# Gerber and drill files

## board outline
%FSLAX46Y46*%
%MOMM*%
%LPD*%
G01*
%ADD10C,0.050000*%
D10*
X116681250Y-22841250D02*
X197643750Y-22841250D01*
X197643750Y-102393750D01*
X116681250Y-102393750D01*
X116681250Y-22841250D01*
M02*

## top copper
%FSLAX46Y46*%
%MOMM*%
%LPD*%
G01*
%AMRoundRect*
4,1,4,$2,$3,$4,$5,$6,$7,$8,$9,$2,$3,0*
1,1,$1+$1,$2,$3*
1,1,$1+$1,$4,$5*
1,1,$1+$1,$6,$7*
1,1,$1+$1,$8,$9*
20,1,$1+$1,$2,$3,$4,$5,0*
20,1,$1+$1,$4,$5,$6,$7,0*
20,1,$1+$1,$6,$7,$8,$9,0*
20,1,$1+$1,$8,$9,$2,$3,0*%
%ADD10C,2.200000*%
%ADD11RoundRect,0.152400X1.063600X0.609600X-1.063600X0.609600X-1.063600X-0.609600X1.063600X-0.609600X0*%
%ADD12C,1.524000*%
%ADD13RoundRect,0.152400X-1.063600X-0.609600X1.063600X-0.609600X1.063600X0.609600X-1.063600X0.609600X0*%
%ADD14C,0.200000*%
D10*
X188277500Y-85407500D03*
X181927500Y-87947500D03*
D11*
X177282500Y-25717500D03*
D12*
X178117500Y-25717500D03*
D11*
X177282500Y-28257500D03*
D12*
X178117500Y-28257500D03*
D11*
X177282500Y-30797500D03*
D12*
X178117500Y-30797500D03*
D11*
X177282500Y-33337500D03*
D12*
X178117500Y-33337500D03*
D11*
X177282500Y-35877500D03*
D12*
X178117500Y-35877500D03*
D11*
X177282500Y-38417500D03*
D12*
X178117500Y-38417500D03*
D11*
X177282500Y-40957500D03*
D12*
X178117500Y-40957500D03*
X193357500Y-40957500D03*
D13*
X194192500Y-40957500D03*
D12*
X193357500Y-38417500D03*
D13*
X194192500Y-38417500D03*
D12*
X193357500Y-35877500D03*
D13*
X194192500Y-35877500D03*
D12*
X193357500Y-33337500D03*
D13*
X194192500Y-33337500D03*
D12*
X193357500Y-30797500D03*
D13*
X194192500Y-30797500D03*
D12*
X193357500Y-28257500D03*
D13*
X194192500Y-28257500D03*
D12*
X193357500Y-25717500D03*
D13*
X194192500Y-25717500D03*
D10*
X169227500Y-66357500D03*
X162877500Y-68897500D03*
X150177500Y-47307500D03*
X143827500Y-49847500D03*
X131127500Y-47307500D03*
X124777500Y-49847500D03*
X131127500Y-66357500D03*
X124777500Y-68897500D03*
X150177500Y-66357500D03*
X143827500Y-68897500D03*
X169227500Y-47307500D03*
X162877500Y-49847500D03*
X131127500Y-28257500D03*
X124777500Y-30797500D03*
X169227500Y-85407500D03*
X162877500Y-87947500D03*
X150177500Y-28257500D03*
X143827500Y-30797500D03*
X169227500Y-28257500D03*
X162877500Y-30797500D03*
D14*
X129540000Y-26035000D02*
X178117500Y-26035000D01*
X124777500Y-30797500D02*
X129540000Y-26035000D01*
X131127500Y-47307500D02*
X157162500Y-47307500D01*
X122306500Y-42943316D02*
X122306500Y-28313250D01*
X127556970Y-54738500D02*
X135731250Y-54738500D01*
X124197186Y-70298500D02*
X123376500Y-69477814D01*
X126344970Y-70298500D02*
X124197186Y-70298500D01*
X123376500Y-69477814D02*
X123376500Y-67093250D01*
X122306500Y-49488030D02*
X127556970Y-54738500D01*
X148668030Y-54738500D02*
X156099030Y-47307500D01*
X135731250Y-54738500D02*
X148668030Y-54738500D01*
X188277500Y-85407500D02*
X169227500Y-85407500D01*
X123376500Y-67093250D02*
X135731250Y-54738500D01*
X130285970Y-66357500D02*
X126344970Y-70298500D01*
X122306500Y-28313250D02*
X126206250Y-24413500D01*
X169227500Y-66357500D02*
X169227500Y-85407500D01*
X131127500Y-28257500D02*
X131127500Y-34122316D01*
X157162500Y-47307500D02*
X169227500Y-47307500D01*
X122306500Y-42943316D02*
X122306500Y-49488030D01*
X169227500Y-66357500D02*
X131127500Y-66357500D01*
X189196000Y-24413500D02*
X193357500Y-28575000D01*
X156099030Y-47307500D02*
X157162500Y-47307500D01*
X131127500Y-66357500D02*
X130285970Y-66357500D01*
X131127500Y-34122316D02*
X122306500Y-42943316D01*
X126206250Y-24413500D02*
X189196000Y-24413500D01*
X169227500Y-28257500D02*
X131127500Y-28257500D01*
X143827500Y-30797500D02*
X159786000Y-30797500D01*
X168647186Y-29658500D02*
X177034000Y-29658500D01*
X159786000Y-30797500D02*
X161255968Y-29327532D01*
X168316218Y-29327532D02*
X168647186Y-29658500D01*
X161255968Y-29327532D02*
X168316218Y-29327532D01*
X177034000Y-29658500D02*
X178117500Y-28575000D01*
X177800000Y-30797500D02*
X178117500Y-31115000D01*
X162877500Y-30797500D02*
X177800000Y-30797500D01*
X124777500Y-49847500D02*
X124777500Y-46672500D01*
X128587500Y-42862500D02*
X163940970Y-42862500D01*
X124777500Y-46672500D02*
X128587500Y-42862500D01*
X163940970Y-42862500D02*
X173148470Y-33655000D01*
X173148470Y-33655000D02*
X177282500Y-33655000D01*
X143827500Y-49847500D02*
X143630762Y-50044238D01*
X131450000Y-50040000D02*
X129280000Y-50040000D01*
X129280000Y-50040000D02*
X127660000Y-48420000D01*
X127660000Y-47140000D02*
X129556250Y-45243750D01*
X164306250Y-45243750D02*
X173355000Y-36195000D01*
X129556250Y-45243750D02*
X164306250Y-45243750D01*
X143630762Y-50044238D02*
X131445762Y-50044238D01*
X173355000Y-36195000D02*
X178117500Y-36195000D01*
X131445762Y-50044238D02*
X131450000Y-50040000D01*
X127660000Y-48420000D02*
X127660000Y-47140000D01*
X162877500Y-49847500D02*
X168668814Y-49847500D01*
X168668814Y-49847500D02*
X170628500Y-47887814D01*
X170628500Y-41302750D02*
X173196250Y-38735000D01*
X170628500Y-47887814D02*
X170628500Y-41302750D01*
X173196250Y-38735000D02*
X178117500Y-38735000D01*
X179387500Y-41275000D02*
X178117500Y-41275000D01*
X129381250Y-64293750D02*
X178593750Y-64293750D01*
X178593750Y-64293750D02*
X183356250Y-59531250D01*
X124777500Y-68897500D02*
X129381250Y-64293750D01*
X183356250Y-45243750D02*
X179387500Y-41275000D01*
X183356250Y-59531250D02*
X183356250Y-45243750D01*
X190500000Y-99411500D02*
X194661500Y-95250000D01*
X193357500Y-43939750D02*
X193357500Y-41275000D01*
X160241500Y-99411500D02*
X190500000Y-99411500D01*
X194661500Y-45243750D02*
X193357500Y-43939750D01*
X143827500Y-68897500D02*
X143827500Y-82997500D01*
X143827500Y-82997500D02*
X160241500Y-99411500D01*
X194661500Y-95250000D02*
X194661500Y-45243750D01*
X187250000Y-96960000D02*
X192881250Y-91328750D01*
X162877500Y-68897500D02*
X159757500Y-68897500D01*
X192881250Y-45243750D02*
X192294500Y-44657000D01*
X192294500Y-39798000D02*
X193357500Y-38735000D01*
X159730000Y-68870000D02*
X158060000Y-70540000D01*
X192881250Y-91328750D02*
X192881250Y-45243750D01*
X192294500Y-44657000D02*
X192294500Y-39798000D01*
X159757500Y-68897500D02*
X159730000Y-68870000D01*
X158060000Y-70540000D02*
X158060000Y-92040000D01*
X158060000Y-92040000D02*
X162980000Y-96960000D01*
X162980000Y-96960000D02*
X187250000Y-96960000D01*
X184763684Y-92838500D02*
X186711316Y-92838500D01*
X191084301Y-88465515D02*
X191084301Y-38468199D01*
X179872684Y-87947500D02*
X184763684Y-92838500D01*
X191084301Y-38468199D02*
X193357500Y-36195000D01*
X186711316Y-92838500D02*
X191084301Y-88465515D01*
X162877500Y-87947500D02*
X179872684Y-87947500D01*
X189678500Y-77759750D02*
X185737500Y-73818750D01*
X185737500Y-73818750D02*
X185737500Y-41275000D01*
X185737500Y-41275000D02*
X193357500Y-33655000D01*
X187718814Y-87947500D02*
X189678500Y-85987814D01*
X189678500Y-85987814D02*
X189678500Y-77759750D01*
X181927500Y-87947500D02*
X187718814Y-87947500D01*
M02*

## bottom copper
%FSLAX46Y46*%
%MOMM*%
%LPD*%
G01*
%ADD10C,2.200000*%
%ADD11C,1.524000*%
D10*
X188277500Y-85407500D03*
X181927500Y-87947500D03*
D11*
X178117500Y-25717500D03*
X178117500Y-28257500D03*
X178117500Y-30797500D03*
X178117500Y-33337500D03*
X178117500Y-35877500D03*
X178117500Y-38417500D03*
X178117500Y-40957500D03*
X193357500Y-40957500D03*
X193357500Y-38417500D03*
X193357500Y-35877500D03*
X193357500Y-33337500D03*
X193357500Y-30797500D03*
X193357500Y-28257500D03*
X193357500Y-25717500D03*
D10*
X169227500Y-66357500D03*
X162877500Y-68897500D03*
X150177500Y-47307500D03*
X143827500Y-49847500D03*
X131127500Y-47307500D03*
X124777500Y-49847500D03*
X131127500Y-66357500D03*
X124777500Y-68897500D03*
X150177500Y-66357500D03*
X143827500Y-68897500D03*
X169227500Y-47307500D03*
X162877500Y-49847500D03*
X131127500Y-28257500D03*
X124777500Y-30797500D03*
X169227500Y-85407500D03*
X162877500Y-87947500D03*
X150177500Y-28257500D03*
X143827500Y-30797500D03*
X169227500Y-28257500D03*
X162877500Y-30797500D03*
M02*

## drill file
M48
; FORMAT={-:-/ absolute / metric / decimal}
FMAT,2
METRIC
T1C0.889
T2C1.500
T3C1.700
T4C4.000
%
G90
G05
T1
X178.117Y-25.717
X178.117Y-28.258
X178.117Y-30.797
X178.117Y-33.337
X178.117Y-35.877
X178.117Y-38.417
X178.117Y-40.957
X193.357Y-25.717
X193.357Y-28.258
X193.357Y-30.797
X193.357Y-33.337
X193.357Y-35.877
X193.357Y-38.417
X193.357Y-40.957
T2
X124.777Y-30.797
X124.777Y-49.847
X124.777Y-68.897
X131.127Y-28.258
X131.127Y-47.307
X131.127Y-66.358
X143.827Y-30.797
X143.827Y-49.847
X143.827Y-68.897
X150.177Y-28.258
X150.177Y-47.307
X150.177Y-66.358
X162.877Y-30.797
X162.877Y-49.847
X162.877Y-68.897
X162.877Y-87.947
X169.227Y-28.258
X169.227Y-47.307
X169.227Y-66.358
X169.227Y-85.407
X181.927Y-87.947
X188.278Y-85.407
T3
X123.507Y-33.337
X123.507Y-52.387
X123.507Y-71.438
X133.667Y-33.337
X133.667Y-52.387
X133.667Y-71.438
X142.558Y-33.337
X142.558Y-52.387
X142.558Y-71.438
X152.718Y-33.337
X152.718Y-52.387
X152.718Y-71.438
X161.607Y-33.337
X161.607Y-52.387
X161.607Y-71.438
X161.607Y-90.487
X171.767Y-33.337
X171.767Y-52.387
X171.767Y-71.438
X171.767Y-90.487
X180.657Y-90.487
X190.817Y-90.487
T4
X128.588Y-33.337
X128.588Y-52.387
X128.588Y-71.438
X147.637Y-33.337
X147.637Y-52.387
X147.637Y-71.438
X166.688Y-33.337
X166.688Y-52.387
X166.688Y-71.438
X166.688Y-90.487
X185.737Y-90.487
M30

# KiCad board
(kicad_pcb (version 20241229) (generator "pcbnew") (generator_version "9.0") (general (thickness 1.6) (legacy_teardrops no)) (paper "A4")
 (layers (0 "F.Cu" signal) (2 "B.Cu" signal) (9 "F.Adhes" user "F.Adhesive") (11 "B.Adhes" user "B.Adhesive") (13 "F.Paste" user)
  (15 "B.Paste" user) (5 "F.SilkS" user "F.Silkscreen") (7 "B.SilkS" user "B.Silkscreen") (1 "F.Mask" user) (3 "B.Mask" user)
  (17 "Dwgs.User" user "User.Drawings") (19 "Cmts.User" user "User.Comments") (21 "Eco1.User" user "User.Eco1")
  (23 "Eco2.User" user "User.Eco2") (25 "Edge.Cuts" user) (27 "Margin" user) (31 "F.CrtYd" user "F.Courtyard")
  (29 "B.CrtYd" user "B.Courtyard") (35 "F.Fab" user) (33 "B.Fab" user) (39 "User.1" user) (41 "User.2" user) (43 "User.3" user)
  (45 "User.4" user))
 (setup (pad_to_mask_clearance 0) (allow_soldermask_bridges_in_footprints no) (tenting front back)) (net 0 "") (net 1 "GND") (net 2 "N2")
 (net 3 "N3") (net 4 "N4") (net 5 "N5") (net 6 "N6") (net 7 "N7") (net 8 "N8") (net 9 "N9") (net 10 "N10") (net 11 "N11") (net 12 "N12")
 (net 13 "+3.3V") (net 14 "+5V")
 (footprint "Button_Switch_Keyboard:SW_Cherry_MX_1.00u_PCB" (layer "F.Cu") (at 188.2775 85.4075)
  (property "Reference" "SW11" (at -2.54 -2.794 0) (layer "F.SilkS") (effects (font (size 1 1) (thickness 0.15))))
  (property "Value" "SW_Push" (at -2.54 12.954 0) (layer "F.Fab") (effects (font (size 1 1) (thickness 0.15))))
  (pad "" np_thru_hole circle (at -7.62 5.08) (size 1.7 1.7) (drill 1.7) (layers "*.Cu" "*.Mask"))
  (pad "" np_thru_hole circle (at -2.54 5.08) (size 4 4) (drill 4) (layers "*.Cu" "*.Mask"))
  (pad "" np_thru_hole circle (at 2.54 5.08) (size 1.7 1.7) (drill 1.7) (layers "*.Cu" "*.Mask"))
  (pad "1" thru_hole circle (at 0 0) (size 2.2 2.2) (drill 1.5) (layers "*.Cu" "*.Mask") (remove_unused_layers no) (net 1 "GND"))
  (pad "2" thru_hole circle (at -6.35 2.54) (size 2.2 2.2) (drill 1.5) (layers "*.Cu" "*.Mask") (remove_unused_layers no) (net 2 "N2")))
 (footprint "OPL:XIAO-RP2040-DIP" (layer "F.Cu") (at 185.7375 33.3375)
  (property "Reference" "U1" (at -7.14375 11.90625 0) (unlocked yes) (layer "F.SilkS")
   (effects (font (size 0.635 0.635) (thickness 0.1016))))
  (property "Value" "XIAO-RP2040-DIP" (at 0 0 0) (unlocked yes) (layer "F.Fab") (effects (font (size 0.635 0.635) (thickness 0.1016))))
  (pad "1" smd roundrect (at -8.455 -7.62 180) (size 2.432 1.524) (layers "F.Cu" "F.Mask") (roundrect_rratio 0.1) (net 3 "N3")
   (thermal_bridge_angle 45))
  (pad "1" thru_hole circle (at -7.62 -7.62 180) (size 1.524 1.524) (drill 0.889) (layers "*.Cu" "*.Mask") (remove_unused_layers no)
   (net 3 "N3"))
  (pad "2" smd roundrect (at -8.455 -5.08 180) (size 2.432 1.524) (layers "F.Cu" "F.Mask") (roundrect_rratio 0.1) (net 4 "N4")
   (thermal_bridge_angle 45))
  (pad "2" thru_hole circle (at -7.62 -5.08 180) (size 1.524 1.524) (drill 0.889) (layers "*.Cu" "*.Mask") (remove_unused_layers no)
   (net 4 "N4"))
  (pad "3" smd roundrect (at -8.455 -2.54 180) (size 2.432 1.524) (layers "F.Cu" "F.Mask") (roundrect_rratio 0.1) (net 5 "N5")
   (thermal_bridge_angle 45))
  (pad "3" thru_hole circle (at -7.62 -2.54 180) (size 1.524 1.524) (drill 0.889) (layers "*.Cu" "*.Mask") (remove_unused_layers no)
   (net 5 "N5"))
  (pad "4" smd roundrect (at -8.455 0 180) (size 2.432 1.524) (layers "F.Cu" "F.Mask") (roundrect_rratio 0.1) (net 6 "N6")
   (thermal_bridge_angle 45))
  (pad "4" thru_hole circle (at -7.62 0 180) (size 1.524 1.524) (drill 0.889) (layers "*.Cu" "*.Mask") (remove_unused_layers no)
   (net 6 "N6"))
  (pad "5" smd roundrect (at -8.455 2.54 180) (size 2.432 1.524) (layers "F.Cu" "F.Mask") (roundrect_rratio 0.1) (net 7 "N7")
   (thermal_bridge_angle 45))
  (pad "5" thru_hole circle (at -7.62 2.54 180) (size 1.524 1.524) (drill 0.889) (layers "*.Cu" "*.Mask") (remove_unused_layers no)
   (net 7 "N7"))
  (pad "6" smd roundrect (at -8.455 5.08 180) (size 2.432 1.524) (layers "F.Cu" "F.Mask") (roundrect_rratio 0.1) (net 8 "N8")
   (thermal_bridge_angle 45))
  (pad "6" thru_hole circle (at -7.62 5.08 180) (size 1.524 1.524) (drill 0.889) (layers "*.Cu" "*.Mask") (remove_unused_layers no)
   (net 8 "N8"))
  (pad "7" smd roundrect (at -8.455 7.62 180) (size 2.432 1.524) (layers "F.Cu" "F.Mask") (roundrect_rratio 0.1) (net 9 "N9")
   (thermal_bridge_angle 45))
  (pad "7" thru_hole circle (at -7.62 7.62 180) (size 1.524 1.524) (drill 0.889) (layers "*.Cu" "*.Mask") (remove_unused_layers no)
   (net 9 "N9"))
  (pad "8" thru_hole circle (at 7.62 7.62) (size 1.524 1.524) (drill 0.889) (layers "*.Cu" "*.Mask") (remove_unused_layers no)
   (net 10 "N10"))
  (pad "8" smd roundrect (at 8.455 7.62) (size 2.432 1.524) (layers "F.Cu" "F.Mask") (roundrect_rratio 0.1) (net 10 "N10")
   (thermal_bridge_angle 45))
  (pad "9" thru_hole circle (at 7.62 5.08) (size 1.524 1.524) (drill 0.889) (layers "*.Cu" "*.Mask") (remove_unused_layers no)
   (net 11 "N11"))
  (pad "9" smd roundrect (at 8.455 5.08) (size 2.432 1.524) (layers "F.Cu" "F.Mask") (roundrect_rratio 0.1) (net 11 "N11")
   (thermal_bridge_angle 45))
  (pad "10" thru_hole circle (at 7.62 2.54) (size 1.524 1.524) (drill 0.889) (layers "*.Cu" "*.Mask") (remove_unused_layers no)
   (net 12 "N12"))
  (pad "10" smd roundrect (at 8.455 2.54) (size 2.432 1.524) (layers "F.Cu" "F.Mask") (roundrect_rratio 0.1) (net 12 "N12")
   (thermal_bridge_angle 45))
  (pad "11" thru_hole circle (at 7.62 0) (size 1.524 1.524) (drill 0.889) (layers "*.Cu" "*.Mask") (remove_unused_layers no) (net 2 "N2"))
  (pad "11" smd roundrect (at 8.455 0) (size 2.432 1.524) (layers "F.Cu" "F.Mask") (roundrect_rratio 0.1) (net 2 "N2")
   (thermal_bridge_angle 45))
  (pad "12" thru_hole circle (at 7.62 -2.54) (size 1.524 1.524) (drill 0.889) (layers "*.Cu" "*.Mask") (remove_unused_layers no)
   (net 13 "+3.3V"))
  (pad "12" smd roundrect (at 8.455 -2.54) (size 2.432 1.524) (layers "F.Cu" "F.Mask") (roundrect_rratio 0.1) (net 13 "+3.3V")
   (thermal_bridge_angle 45))
  (pad "13" thru_hole circle (at 7.62 -5.08) (size 1.524 1.524) (drill 0.889) (layers "*.Cu" "*.Mask") (remove_unused_layers no)
   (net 1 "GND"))
  (pad "13" smd roundrect (at 8.455 -5.08) (size 2.432 1.524) (layers "F.Cu" "F.Mask") (roundrect_rratio 0.1) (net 1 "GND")
   (thermal_bridge_angle 45))
  (pad "14" thru_hole circle (at 7.62 -7.62) (size 1.524 1.524) (drill 0.889) (layers "*.Cu" "*.Mask") (remove_unused_layers no)
   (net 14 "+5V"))
  (pad "14" smd roundrect (at 8.455 -7.62) (size 2.432 1.524) (layers "F.Cu" "F.Mask") (roundrect_rratio 0.1) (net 14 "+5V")
   (thermal_bridge_angle 45)))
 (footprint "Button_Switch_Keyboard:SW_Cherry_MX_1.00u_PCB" (layer "F.Cu") (at 169.2275 66.3575)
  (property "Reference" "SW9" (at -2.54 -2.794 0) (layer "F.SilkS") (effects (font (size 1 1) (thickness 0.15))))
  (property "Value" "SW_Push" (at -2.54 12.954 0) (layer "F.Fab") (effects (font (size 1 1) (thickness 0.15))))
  (pad "" np_thru_hole circle (at -7.62 5.08) (size 1.7 1.7) (drill 1.7) (layers "*.Cu" "*.Mask"))
  (pad "" np_thru_hole circle (at -2.54 5.08) (size 4 4) (drill 4) (layers "*.Cu" "*.Mask"))
  (pad "" np_thru_hole circle (at 2.54 5.08) (size 1.7 1.7) (drill 1.7) (layers "*.Cu" "*.Mask"))
  (pad "1" thru_hole circle (at 0 0) (size 2.2 2.2) (drill 1.5) (layers "*.Cu" "*.Mask") (remove_unused_layers no) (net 1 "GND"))
  (pad "2" thru_hole circle (at -6.35 2.54) (size 2.2 2.2) (drill 1.5) (layers "*.Cu" "*.Mask") (remove_unused_layers no) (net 11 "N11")))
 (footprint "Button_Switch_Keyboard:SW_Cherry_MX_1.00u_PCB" (layer "F.Cu") (at 150.1775 47.3075)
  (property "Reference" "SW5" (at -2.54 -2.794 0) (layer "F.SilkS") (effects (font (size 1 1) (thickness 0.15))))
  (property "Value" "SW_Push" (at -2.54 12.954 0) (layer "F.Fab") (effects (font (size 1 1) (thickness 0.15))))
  (pad "" np_thru_hole circle (at -7.62 5.08) (size 1.7 1.7) (drill 1.7) (layers "*.Cu" "*.Mask"))
  (pad "" np_thru_hole circle (at -2.54 5.08) (size 4 4) (drill 4) (layers "*.Cu" "*.Mask"))
  (pad "" np_thru_hole circle (at 2.54 5.08) (size 1.7 1.7) (drill 1.7) (layers "*.Cu" "*.Mask"))
  (pad "1" thru_hole circle (at 0 0) (size 2.2 2.2) (drill 1.5) (layers "*.Cu" "*.Mask") (remove_unused_layers no) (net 1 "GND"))
  (pad "2" thru_hole circle (at -6.35 2.54) (size 2.2 2.2) (drill 1.5) (layers "*.Cu" "*.Mask") (remove_unused_layers no) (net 7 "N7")))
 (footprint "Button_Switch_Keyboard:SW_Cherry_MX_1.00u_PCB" (layer "F.Cu") (at 131.1275 47.3075)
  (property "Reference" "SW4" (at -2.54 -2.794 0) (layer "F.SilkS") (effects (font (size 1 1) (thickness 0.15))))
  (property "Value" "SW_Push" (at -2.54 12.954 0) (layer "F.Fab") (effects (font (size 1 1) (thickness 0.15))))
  (pad "" np_thru_hole circle (at -7.62 5.08) (size 1.7 1.7) (drill 1.7) (layers "*.Cu" "*.Mask"))
  (pad "" np_thru_hole circle (at -2.54 5.08) (size 4 4) (drill 4) (layers "*.Cu" "*.Mask"))
  (pad "" np_thru_hole circle (at 2.54 5.08) (size 1.7 1.7) (drill 1.7) (layers "*.Cu" "*.Mask"))
  (pad "1" thru_hole circle (at 0 0) (size 2.2 2.2) (drill 1.5) (layers "*.Cu" "*.Mask") (remove_unused_layers no) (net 1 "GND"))
  (pad "2" thru_hole circle (at -6.35 2.54) (size 2.2 2.2) (drill 1.5) (layers "*.Cu" "*.Mask") (remove_unused_layers no) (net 6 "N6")))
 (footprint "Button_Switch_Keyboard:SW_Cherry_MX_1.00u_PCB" (layer "F.Cu") (at 131.1275 66.3575)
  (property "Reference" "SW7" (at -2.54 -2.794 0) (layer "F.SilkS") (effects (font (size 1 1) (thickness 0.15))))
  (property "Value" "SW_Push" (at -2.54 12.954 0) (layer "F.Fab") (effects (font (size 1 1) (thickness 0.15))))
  (pad "" np_thru_hole circle (at -7.62 5.08) (size 1.7 1.7) (drill 1.7) (layers "*.Cu" "*.Mask"))
  (pad "" np_thru_hole circle (at -2.54 5.08) (size 4 4) (drill 4) (layers "*.Cu" "*.Mask"))
  (pad "" np_thru_hole circle (at 2.54 5.08) (size 1.7 1.7) (drill 1.7) (layers "*.Cu" "*.Mask"))
  (pad "1" thru_hole circle (at 0 0) (size 2.2 2.2) (drill 1.5) (layers "*.Cu" "*.Mask") (remove_unused_layers no) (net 1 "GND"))
  (pad "2" thru_hole circle (at -6.35 2.54) (size 2.2 2.2) (drill 1.5) (layers "*.Cu" "*.Mask") (remove_unused_layers no) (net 9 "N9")))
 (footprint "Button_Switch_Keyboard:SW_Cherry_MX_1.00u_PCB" (layer "F.Cu") (at 150.1775 66.3575)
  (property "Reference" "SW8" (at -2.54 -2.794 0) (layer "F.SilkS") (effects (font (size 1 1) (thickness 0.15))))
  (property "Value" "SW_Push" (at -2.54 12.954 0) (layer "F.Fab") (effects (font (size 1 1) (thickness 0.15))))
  (pad "" np_thru_hole circle (at -7.62 5.08) (size 1.7 1.7) (drill 1.7) (layers "*.Cu" "*.Mask"))
  (pad "" np_thru_hole circle (at -2.54 5.08) (size 4 4) (drill 4) (layers "*.Cu" "*.Mask"))
  (pad "" np_thru_hole circle (at 2.54 5.08) (size 1.7 1.7) (drill 1.7) (layers "*.Cu" "*.Mask"))
  (pad "1" thru_hole circle (at 0 0) (size 2.2 2.2) (drill 1.5) (layers "*.Cu" "*.Mask") (remove_unused_layers no) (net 1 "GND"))
  (pad "2" thru_hole circle (at -6.35 2.54) (size 2.2 2.2) (drill 1.5) (layers "*.Cu" "*.Mask") (remove_unused_layers no) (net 10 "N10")))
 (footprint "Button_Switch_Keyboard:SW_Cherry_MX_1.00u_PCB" (layer "F.Cu") (at 169.2275 47.3075)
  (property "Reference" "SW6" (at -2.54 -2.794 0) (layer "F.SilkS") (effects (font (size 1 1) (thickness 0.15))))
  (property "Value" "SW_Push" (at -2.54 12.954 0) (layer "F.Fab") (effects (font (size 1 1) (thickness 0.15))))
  (pad "" np_thru_hole circle (at -7.62 5.08) (size 1.7 1.7) (drill 1.7) (layers "*.Cu" "*.Mask"))
  (pad "" np_thru_hole circle (at -2.54 5.08) (size 4 4) (drill 4) (layers "*.Cu" "*.Mask"))
  (pad "" np_thru_hole circle (at 2.54 5.08) (size 1.7 1.7) (drill 1.7) (layers "*.Cu" "*.Mask"))
  (pad "1" thru_hole circle (at 0 0) (size 2.2 2.2) (drill 1.5) (layers "*.Cu" "*.Mask") (remove_unused_layers no) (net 1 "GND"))
  (pad "2" thru_hole circle (at -6.35 2.54) (size 2.2 2.2) (drill 1.5) (layers "*.Cu" "*.Mask") (remove_unused_layers no) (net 8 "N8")))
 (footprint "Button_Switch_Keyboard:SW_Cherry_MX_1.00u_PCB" (layer "F.Cu") (at 131.1275 28.2575)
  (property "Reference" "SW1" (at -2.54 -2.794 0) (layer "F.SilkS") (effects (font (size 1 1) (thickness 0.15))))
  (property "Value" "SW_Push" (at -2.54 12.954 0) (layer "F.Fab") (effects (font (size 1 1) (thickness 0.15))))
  (pad "" np_thru_hole circle (at -7.62 5.08) (size 1.7 1.7) (drill 1.7) (layers "*.Cu" "*.Mask"))
  (pad "" np_thru_hole circle (at -2.54 5.08) (size 4 4) (drill 4) (layers "*.Cu" "*.Mask"))
  (pad "" np_thru_hole circle (at 2.54 5.08) (size 1.7 1.7) (drill 1.7) (layers "*.Cu" "*.Mask"))
  (pad "1" thru_hole circle (at 0 0) (size 2.2 2.2) (drill 1.5) (layers "*.Cu" "*.Mask") (remove_unused_layers no) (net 1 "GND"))
  (pad "2" thru_hole circle (at -6.35 2.54) (size 2.2 2.2) (drill 1.5) (layers "*.Cu" "*.Mask") (remove_unused_layers no) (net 3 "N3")))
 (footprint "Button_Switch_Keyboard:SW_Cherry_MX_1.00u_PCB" (layer "F.Cu") (at 169.2275 85.4075)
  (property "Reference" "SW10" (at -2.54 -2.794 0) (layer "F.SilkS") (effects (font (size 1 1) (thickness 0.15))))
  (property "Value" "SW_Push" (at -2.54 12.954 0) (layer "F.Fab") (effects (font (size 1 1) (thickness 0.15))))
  (pad "" np_thru_hole circle (at -7.62 5.08) (size 1.7 1.7) (drill 1.7) (layers "*.Cu" "*.Mask"))
  (pad "" np_thru_hole circle (at -2.54 5.08) (size 4 4) (drill 4) (layers "*.Cu" "*.Mask"))
  (pad "" np_thru_hole circle (at 2.54 5.08) (size 1.7 1.7) (drill 1.7) (layers "*.Cu" "*.Mask"))
  (pad "1" thru_hole circle (at 0 0) (size 2.2 2.2) (drill 1.5) (layers "*.Cu" "*.Mask") (remove_unused_layers no) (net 1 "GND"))
  (pad "2" thru_hole circle (at -6.35 2.54) (size 2.2 2.2) (drill 1.5) (layers "*.Cu" "*.Mask") (remove_unused_layers no) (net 12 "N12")))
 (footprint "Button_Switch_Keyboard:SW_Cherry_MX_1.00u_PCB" (layer "F.Cu") (at 150.1775 28.2575)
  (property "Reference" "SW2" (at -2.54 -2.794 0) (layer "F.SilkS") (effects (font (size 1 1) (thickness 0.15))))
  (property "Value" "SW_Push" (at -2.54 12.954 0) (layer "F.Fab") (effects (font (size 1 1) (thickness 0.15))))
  (pad "" np_thru_hole circle (at -7.62 5.08) (size 1.7 1.7) (drill 1.7) (layers "*.Cu" "*.Mask"))
  (pad "" np_thru_hole circle (at -2.54 5.08) (size 4 4) (drill 4) (layers "*.Cu" "*.Mask"))
  (pad "" np_thru_hole circle (at 2.54 5.08) (size 1.7 1.7) (drill 1.7) (layers "*.Cu" "*.Mask"))
  (pad "1" thru_hole circle (at 0 0) (size 2.2 2.2) (drill 1.5) (layers "*.Cu" "*.Mask") (remove_unused_layers no) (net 1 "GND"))
  (pad "2" thru_hole circle (at -6.35 2.54) (size 2.2 2.2) (drill 1.5) (layers "*.Cu" "*.Mask") (remove_unused_layers no) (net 4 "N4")))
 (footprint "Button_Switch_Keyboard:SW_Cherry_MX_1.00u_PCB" (layer "F.Cu") (at 169.2275 28.2575)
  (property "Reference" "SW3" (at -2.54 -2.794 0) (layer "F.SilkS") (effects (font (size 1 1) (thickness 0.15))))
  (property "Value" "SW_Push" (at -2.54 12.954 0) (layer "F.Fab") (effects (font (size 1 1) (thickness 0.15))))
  (pad "" np_thru_hole circle (at -7.62 5.08) (size 1.7 1.7) (drill 1.7) (layers "*.Cu" "*.Mask"))
  (pad "" np_thru_hole circle (at -2.54 5.08) (size 4 4) (drill 4) (layers "*.Cu" "*.Mask"))
  (pad "" np_thru_hole circle (at 2.54 5.08) (size 1.7 1.7) (drill 1.7) (layers "*.Cu" "*.Mask"))
  (pad "1" thru_hole circle (at 0 0) (size 2.2 2.2) (drill 1.5) (layers "*.Cu" "*.Mask") (remove_unused_layers no) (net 1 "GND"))
  (pad "2" thru_hole circle (at -6.35 2.54) (size 2.2 2.2) (drill 1.5) (layers "*.Cu" "*.Mask") (remove_unused_layers no) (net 5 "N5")))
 (gr_rect (start 116.68125 22.84125) (end 197.64375 102.39375) (stroke (width 0.05) (type default)) (fill no) (layer "Edge.Cuts"))
 (segment (start 129.54 26.035) (end 178.1175 26.035) (width 0.2) (layer "F.Cu") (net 3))
 (segment (start 124.7775 30.7975) (end 129.54 26.035) (width 0.2) (layer "F.Cu") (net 3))
 (segment (start 131.1275 47.3075) (end 157.1625 47.3075) (width 0.2) (layer "F.Cu") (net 1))
 (segment (start 122.3065 42.943316) (end 122.3065 28.31325) (width 0.2) (layer "F.Cu") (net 1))
 (segment (start 127.55697 54.7385) (end 135.73125 54.7385) (width 0.2) (layer "F.Cu") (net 1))
 (segment (start 124.197186 70.2985) (end 123.3765 69.477814) (width 0.2) (layer "F.Cu") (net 1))
 (segment (start 126.34497 70.2985) (end 124.197186 70.2985) (width 0.2) (layer "F.Cu") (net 1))
 (segment (start 123.3765 69.477814) (end 123.3765 67.09325) (width 0.2) (layer "F.Cu") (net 1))
 (segment (start 122.3065 49.48803) (end 127.55697 54.7385) (width 0.2) (layer "F.Cu") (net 1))
 (segment (start 148.66803 54.7385) (end 156.09903 47.3075) (width 0.2) (layer "F.Cu") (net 1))
 (segment (start 135.73125 54.7385) (end 148.66803 54.7385) (width 0.2) (layer "F.Cu") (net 1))
 (segment (start 188.2775 85.4075) (end 169.2275 85.4075) (width 0.2) (layer "F.Cu") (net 1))
 (segment (start 123.3765 67.09325) (end 135.73125 54.7385) (width 0.2) (layer "F.Cu") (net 1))
 (segment (start 130.28597 66.3575) (end 126.34497 70.2985) (width 0.2) (layer "F.Cu") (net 1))
 (segment (start 122.3065 28.31325) (end 126.20625 24.4135) (width 0.2) (layer "F.Cu") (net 1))
 (segment (start 169.2275 66.3575) (end 169.2275 85.4075) (width 0.2) (layer "F.Cu") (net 1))
 (segment (start 131.1275 28.2575) (end 131.1275 34.122316) (width 0.2) (layer "F.Cu") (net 1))
 (segment (start 157.1625 47.3075) (end 169.2275 47.3075) (width 0.2) (layer "F.Cu") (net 1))
 (segment (start 122.3065 42.943316) (end 122.3065 49.48803) (width 0.2) (layer "F.Cu") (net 1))
 (segment (start 169.2275 66.3575) (end 131.1275 66.3575) (width 0.2) (layer "F.Cu") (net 1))
 (segment (start 189.196 24.4135) (end 193.3575 28.575) (width 0.2) (layer "F.Cu") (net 1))
 (segment (start 156.09903 47.3075) (end 157.1625 47.3075) (width 0.2) (layer "F.Cu") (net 1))
 (segment (start 131.1275 66.3575) (end 130.28597 66.3575) (width 0.2) (layer "F.Cu") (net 1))
 (segment (start 131.1275 34.122316) (end 122.3065 42.943316) (width 0.2) (layer "F.Cu") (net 1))
 (segment (start 126.20625 24.4135) (end 189.196 24.4135) (width 0.2) (layer "F.Cu") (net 1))
 (segment (start 169.2275 28.2575) (end 131.1275 28.2575) (width 0.2) (layer "F.Cu") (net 1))
 (segment (start 143.8275 30.7975) (end 159.786 30.7975) (width 0.2) (layer "F.Cu") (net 4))
 (segment (start 168.647186 29.6585) (end 177.034 29.6585) (width 0.2) (layer "F.Cu") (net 4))
 (segment (start 159.786 30.7975) (end 161.255968 29.327532) (width 0.2) (layer "F.Cu") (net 4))
 (segment (start 168.316218 29.327532) (end 168.647186 29.6585) (width 0.2) (layer "F.Cu") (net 4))
 (segment (start 161.255968 29.327532) (end 168.316218 29.327532) (width 0.2) (layer "F.Cu") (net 4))
 (segment (start 177.034 29.6585) (end 178.1175 28.575) (width 0.2) (layer "F.Cu") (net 4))
 (segment (start 177.8 30.7975) (end 178.1175 31.115) (width 0.2) (layer "F.Cu") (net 5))
 (segment (start 162.8775 30.7975) (end 177.8 30.7975) (width 0.2) (layer "F.Cu") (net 5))
 (segment (start 124.7775 49.8475) (end 124.7775 46.6725) (width 0.2) (layer "F.Cu") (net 6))
 (segment (start 128.5875 42.8625) (end 163.94097 42.8625) (width 0.2) (layer "F.Cu") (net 6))
 (segment (start 124.7775 46.6725) (end 128.5875 42.8625) (width 0.2) (layer "F.Cu") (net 6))
 (segment (start 163.94097 42.8625) (end 173.14847 33.655) (width 0.2) (layer "F.Cu") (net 6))
 (segment (start 173.14847 33.655) (end 177.2825 33.655) (width 0.2) (layer "F.Cu") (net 6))
 (segment (start 143.8275 49.8475) (end 143.630762 50.044238) (width 0.2) (layer "F.Cu") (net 7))
 (segment (start 131.45 50.04) (end 129.28 50.04) (width 0.2) (layer "F.Cu") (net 7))
 (segment (start 129.28 50.04) (end 127.66 48.42) (width 0.2) (layer "F.Cu") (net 7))
 (segment (start 127.66 47.14) (end 129.55625 45.24375) (width 0.2) (layer "F.Cu") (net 7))
 (segment (start 164.30625 45.24375) (end 173.355 36.195) (width 0.2) (layer "F.Cu") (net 7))
 (segment (start 129.55625 45.24375) (end 164.30625 45.24375) (width 0.2) (layer "F.Cu") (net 7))
 (segment (start 143.630762 50.044238) (end 131.445762 50.044238) (width 0.2) (layer "F.Cu") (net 7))
 (segment (start 173.355 36.195) (end 178.1175 36.195) (width 0.2) (layer "F.Cu") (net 7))
 (segment (start 131.445762 50.044238) (end 131.45 50.04) (width 0.2) (layer "F.Cu") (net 7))
 (segment (start 127.66 48.42) (end 127.66 47.14) (width 0.2) (layer "F.Cu") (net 7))
 (segment (start 162.8775 49.8475) (end 168.668814 49.8475) (width 0.2) (layer "F.Cu") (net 8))
 (segment (start 168.668814 49.8475) (end 170.6285 47.887814) (width 0.2) (layer "F.Cu") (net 8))
 (segment (start 170.6285 41.30275) (end 173.19625 38.735) (width 0.2) (layer "F.Cu") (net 8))
 (segment (start 170.6285 47.887814) (end 170.6285 41.30275) (width 0.2) (layer "F.Cu") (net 8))
 (segment (start 173.19625 38.735) (end 178.1175 38.735) (width 0.2) (layer "F.Cu") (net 8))
 (segment (start 179.3875 41.275) (end 178.1175 41.275) (width 0.2) (layer "F.Cu") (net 9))
 (segment (start 129.38125 64.29375) (end 178.59375 64.29375) (width 0.2) (layer "F.Cu") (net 9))
 (segment (start 178.59375 64.29375) (end 183.35625 59.53125) (width 0.2) (layer "F.Cu") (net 9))
 (segment (start 124.7775 68.8975) (end 129.38125 64.29375) (width 0.2) (layer "F.Cu") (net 9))
 (segment (start 183.35625 45.24375) (end 179.3875 41.275) (width 0.2) (layer "F.Cu") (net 9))
 (segment (start 183.35625 59.53125) (end 183.35625 45.24375) (width 0.2) (layer "F.Cu") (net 9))
 (segment (start 190.5 99.4115) (end 194.6615 95.25) (width 0.2) (layer "F.Cu") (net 10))
 (segment (start 193.3575 43.93975) (end 193.3575 41.275) (width 0.2) (layer "F.Cu") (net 10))
 (segment (start 160.2415 99.4115) (end 190.5 99.4115) (width 0.2) (layer "F.Cu") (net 10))
 (segment (start 194.6615 45.24375) (end 193.3575 43.93975) (width 0.2) (layer "F.Cu") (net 10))
 (segment (start 143.8275 68.8975) (end 143.8275 82.9975) (width 0.2) (layer "F.Cu") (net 10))
 (segment (start 143.8275 82.9975) (end 160.2415 99.4115) (width 0.2) (layer "F.Cu") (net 10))
 (segment (start 194.6615 95.25) (end 194.6615 45.24375) (width 0.2) (layer "F.Cu") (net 10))
 (segment (start 187.25 96.96) (end 192.88125 91.32875) (width 0.2) (layer "F.Cu") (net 11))
 (segment (start 162.8775 68.8975) (end 159.7575 68.8975) (width 0.2) (layer "F.Cu") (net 11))
 (segment (start 192.88125 45.24375) (end 192.2945 44.657) (width 0.2) (layer "F.Cu") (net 11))
 (segment (start 192.2945 39.798) (end 193.3575 38.735) (width 0.2) (layer "F.Cu") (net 11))
 (segment (start 159.73 68.87) (end 158.06 70.54) (width 0.2) (layer "F.Cu") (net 11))
 (segment (start 192.88125 91.32875) (end 192.88125 45.24375) (width 0.2) (layer "F.Cu") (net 11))
 (segment (start 192.2945 44.657) (end 192.2945 39.798) (width 0.2) (layer "F.Cu") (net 11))
 (segment (start 159.7575 68.8975) (end 159.73 68.87) (width 0.2) (layer "F.Cu") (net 11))
 (segment (start 158.06 70.54) (end 158.06 92.04) (width 0.2) (layer "F.Cu") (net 11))
 (segment (start 158.06 92.04) (end 162.98 96.96) (width 0.2) (layer "F.Cu") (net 11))
 (segment (start 162.98 96.96) (end 187.25 96.96) (width 0.2) (layer "F.Cu") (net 11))
 (segment (start 184.763684 92.8385) (end 186.711316 92.8385) (width 0.2) (layer "F.Cu") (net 12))
 (segment (start 191.084301 88.465515) (end 191.084301 38.468199) (width 0.2) (layer "F.Cu") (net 12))
 (segment (start 179.872684 87.9475) (end 184.763684 92.8385) (width 0.2) (layer "F.Cu") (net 12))
 (segment (start 191.084301 38.468199) (end 193.3575 36.195) (width 0.2) (layer "F.Cu") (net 12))
 (segment (start 186.711316 92.8385) (end 191.084301 88.465515) (width 0.2) (layer "F.Cu") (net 12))
 (segment (start 162.8775 87.9475) (end 179.872684 87.9475) (width 0.2) (layer "F.Cu") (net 12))
 (segment (start 189.6785 77.75975) (end 185.7375 73.81875) (width 0.2) (layer "F.Cu") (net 2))
 (segment (start 185.7375 73.81875) (end 185.7375 41.275) (width 0.2) (layer "F.Cu") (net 2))
 (segment (start 185.7375 41.275) (end 193.3575 33.655) (width 0.2) (layer "F.Cu") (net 2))
 (segment (start 187.718814 87.9475) (end 189.6785 85.987814) (width 0.2) (layer "F.Cu") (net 2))
 (segment (start 189.6785 85.987814) (end 189.6785 77.75975) (width 0.2) (layer "F.Cu") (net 2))
 (segment (start 181.9275 87.9475) (end 187.718814 87.9475) (width 0.2) (layer "F.Cu") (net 2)))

